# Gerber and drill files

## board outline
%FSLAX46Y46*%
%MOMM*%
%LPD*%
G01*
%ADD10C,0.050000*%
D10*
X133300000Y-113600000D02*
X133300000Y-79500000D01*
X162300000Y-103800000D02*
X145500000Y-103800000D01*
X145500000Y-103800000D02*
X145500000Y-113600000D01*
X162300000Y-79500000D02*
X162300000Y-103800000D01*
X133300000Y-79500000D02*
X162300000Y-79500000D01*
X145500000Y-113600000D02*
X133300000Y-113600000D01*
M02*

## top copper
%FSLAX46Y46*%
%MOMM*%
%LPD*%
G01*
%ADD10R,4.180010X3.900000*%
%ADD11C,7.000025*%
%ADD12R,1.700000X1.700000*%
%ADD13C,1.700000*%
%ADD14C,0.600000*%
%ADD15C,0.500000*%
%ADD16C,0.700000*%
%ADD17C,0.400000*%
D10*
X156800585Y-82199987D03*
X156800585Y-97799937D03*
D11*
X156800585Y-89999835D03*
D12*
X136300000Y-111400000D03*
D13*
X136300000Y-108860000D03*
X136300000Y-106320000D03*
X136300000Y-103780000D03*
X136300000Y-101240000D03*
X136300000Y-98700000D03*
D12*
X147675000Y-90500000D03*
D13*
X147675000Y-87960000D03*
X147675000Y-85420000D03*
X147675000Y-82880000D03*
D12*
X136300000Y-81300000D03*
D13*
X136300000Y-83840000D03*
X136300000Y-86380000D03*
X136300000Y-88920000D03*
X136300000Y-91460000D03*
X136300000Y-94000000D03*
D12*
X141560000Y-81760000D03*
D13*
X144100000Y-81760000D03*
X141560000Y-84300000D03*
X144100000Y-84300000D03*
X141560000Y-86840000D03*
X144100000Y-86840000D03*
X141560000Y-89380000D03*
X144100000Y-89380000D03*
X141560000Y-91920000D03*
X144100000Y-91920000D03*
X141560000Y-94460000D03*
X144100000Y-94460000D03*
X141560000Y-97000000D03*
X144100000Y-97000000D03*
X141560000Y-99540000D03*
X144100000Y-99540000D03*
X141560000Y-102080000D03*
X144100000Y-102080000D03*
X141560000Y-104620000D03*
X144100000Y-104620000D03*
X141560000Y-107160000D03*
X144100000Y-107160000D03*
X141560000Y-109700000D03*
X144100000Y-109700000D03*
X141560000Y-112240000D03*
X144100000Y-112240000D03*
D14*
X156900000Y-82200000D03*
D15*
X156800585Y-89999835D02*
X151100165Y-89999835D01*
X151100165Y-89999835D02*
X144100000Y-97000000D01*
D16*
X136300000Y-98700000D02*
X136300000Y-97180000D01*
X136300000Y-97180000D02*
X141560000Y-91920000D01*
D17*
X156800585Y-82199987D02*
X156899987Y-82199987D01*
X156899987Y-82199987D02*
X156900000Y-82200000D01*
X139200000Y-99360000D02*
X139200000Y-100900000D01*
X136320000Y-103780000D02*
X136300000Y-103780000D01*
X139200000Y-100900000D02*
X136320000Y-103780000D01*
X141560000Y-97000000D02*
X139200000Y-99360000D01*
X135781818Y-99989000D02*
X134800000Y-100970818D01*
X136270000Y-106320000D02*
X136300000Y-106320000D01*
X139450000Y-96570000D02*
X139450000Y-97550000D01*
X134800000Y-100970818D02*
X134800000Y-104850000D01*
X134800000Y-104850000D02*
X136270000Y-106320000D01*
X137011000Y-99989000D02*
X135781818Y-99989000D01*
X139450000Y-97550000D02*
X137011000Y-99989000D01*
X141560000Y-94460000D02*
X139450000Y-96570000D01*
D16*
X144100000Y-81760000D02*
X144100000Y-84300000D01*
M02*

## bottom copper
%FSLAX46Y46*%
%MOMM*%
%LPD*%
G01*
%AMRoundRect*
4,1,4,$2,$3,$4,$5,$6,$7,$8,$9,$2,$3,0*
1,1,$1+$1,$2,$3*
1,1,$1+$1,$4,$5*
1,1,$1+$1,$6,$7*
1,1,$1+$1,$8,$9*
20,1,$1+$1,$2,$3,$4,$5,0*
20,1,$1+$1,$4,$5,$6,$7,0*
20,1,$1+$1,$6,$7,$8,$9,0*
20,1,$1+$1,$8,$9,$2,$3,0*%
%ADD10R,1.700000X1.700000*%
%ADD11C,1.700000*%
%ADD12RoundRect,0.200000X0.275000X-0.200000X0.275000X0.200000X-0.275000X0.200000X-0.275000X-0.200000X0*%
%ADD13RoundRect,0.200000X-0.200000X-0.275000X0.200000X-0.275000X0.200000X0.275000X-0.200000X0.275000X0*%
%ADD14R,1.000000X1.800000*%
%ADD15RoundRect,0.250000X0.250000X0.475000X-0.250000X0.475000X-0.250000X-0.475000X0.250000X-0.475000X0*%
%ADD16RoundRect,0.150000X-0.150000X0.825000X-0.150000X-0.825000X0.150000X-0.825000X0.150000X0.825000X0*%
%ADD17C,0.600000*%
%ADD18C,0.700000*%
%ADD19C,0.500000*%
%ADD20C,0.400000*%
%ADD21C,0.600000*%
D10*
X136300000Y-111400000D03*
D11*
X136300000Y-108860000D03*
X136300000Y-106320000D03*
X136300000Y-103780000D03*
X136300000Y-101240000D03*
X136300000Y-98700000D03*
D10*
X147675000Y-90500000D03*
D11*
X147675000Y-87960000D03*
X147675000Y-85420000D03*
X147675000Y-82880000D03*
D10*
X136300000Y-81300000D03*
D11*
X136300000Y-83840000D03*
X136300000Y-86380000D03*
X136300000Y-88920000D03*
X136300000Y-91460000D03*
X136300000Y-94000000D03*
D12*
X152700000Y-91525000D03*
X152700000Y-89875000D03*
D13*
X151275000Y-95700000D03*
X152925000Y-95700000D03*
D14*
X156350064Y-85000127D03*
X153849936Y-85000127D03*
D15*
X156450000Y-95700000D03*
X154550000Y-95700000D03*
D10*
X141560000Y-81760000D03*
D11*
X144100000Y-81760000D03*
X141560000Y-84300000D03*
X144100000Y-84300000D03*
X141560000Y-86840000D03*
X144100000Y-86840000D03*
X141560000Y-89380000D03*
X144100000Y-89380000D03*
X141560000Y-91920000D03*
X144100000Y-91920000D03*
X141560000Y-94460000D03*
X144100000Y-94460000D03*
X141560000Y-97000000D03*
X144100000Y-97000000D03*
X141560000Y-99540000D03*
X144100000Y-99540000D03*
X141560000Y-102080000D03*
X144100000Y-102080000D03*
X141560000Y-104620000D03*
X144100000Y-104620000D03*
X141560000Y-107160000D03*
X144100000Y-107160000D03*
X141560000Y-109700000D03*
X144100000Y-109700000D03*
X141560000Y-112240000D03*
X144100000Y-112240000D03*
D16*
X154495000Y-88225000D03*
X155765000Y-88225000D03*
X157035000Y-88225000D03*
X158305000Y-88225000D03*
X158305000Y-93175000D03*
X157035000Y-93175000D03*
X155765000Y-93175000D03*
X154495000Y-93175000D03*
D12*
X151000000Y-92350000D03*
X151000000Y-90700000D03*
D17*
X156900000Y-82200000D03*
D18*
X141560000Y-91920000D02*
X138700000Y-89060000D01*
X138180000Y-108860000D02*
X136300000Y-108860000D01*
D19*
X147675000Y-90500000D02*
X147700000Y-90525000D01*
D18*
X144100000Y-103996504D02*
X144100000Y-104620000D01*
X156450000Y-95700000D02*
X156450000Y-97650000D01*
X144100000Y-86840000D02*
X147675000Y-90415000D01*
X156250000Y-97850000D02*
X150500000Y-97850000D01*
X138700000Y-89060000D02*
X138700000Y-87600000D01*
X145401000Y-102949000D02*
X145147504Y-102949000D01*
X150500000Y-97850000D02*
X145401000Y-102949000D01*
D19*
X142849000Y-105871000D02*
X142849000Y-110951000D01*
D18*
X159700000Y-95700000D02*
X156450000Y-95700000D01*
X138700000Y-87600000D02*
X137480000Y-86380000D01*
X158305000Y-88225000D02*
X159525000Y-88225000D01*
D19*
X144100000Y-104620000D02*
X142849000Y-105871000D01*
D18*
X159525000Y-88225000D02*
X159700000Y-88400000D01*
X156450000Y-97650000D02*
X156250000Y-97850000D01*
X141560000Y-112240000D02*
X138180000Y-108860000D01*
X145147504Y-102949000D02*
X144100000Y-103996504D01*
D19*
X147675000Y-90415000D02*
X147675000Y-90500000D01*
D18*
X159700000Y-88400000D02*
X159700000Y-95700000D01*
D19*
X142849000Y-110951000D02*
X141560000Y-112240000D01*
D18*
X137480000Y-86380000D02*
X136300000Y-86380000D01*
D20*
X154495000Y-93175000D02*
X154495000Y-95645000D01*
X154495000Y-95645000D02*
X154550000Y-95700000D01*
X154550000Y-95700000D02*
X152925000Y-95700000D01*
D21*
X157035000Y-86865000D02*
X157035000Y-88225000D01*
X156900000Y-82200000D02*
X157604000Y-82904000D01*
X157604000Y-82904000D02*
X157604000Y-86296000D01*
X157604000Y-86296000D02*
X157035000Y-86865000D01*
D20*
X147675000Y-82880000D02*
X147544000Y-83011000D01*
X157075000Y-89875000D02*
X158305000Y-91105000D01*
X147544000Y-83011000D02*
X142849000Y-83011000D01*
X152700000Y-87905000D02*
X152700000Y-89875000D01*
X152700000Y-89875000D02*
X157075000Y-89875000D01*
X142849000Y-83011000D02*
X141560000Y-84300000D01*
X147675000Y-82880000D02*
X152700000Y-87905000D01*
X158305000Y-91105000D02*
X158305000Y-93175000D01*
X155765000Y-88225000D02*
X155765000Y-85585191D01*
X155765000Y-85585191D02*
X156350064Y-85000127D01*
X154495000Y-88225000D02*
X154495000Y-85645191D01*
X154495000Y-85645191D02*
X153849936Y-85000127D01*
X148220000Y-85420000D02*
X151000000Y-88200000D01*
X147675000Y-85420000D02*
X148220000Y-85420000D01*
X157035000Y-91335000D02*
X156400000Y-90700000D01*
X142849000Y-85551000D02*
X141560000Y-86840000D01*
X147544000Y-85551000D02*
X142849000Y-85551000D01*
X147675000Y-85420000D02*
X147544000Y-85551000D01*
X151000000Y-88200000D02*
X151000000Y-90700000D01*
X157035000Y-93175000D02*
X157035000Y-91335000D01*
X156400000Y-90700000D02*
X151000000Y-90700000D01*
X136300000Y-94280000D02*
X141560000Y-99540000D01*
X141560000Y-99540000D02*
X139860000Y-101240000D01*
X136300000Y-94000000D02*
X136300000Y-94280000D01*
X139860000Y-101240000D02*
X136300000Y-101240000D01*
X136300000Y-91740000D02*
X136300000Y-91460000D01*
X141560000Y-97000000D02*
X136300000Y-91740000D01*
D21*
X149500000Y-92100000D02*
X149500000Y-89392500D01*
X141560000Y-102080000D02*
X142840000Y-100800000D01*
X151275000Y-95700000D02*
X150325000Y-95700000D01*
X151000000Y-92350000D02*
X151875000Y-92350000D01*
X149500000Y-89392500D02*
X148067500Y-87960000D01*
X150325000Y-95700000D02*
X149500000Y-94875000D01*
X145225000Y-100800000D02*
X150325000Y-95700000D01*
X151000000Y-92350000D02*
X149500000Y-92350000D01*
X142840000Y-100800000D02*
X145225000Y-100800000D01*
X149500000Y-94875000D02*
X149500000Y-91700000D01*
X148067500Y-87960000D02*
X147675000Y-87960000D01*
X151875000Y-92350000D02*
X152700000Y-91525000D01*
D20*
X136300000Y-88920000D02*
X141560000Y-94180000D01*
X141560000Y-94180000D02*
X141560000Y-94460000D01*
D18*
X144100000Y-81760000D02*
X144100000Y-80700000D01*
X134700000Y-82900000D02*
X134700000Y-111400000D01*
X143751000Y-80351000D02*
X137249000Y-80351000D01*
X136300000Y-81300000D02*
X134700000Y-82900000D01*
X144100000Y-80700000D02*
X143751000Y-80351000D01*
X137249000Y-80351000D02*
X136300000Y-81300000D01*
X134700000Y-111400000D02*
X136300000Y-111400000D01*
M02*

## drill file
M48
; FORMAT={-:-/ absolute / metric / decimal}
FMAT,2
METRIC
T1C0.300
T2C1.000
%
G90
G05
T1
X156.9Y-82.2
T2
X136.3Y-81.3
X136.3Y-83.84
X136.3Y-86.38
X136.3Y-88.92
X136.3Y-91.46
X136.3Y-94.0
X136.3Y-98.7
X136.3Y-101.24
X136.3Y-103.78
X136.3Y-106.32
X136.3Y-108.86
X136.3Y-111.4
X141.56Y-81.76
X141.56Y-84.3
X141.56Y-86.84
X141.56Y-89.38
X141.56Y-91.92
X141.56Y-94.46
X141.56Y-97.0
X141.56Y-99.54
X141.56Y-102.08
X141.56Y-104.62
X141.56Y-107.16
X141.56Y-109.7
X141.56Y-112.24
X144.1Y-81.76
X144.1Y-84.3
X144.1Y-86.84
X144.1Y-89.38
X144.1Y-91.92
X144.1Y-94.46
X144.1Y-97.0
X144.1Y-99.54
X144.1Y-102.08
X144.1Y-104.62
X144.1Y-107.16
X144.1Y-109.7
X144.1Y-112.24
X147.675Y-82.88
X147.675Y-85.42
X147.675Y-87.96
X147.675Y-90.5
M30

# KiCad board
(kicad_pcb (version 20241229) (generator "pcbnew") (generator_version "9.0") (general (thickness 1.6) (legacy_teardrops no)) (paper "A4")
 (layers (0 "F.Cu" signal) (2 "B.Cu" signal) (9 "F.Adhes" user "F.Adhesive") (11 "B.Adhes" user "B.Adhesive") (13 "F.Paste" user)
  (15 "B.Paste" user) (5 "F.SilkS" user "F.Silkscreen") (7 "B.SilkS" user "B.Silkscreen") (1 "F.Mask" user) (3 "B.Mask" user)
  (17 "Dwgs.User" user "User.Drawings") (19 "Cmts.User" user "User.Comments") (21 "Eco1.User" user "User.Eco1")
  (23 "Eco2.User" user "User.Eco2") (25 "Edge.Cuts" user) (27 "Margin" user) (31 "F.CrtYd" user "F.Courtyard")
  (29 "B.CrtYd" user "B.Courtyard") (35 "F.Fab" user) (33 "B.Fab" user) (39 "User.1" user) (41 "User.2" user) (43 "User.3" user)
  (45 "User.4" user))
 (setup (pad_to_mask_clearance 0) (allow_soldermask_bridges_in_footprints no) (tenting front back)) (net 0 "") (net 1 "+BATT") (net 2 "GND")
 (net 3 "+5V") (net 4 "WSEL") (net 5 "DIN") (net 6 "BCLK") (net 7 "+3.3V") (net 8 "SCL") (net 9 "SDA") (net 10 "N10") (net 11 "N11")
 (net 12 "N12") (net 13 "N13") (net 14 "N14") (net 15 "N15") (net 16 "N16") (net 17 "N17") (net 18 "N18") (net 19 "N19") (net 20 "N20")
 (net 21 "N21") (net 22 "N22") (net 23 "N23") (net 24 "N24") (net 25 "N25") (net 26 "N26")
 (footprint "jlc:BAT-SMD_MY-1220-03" (layer "F.Cu") (at 156.800585 89.999962 -90)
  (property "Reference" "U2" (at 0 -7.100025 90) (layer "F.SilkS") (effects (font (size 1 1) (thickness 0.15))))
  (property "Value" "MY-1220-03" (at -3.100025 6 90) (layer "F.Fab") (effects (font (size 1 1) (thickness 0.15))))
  (pad "1" smd rect (at -7.799975 0 270) (size 3.9 4.18001) (layers "F.Cu" "F.Mask" "F.Paste") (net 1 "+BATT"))
  (pad "2" smd rect (at 7.799975 0 270) (size 3.9 4.18001) (layers "F.Cu" "F.Mask" "F.Paste") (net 1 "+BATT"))
  (pad "3" smd circle (at -0.000127 0 270) (size 7.000025 7.000025) (layers "F.Cu" "F.Mask" "F.Paste") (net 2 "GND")))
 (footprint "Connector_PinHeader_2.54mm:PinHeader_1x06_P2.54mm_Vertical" (layer "F.Cu") (at 136.3 111.4 180)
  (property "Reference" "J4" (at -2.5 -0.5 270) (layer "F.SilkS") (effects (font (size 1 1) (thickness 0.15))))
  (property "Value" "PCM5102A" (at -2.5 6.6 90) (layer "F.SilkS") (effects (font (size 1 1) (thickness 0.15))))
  (pad "1" thru_hole rect (at 0 0 180) (size 1.7 1.7) (drill 1) (layers "*.Cu" "*.Mask") (remove_unused_layers no) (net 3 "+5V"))
  (pad "2" thru_hole circle (at 0 2.54 180) (size 1.7 1.7) (drill 1) (layers "*.Cu" "*.Mask") (remove_unused_layers no) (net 2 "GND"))
  (pad "3" thru_hole circle (at 0 5.08 180) (size 1.7 1.7) (drill 1) (layers "*.Cu" "*.Mask") (remove_unused_layers no) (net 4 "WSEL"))
  (pad "4" thru_hole circle (at 0 7.62 180) (size 1.7 1.7) (drill 1) (layers "*.Cu" "*.Mask") (remove_unused_layers no) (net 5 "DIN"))
  (pad "5" thru_hole circle (at 0 10.16 180) (size 1.7 1.7) (drill 1) (layers "*.Cu" "*.Mask") (remove_unused_layers no) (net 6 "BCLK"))
  (pad "6" thru_hole circle (at 0 12.7 180) (size 1.7 1.7) (drill 1) (layers "*.Cu" "*.Mask") (remove_unused_layers no) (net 2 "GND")))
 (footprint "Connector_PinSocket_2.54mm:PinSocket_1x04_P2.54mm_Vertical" (layer "F.Cu") (at 147.675 90.5 180)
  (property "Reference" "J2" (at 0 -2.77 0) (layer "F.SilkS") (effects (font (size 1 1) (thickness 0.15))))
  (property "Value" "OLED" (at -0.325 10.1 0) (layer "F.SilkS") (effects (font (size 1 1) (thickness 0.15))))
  (pad "1" thru_hole rect (at 0 0 180) (size 1.7 1.7) (drill 1) (layers "*.Cu" "*.Mask") (remove_unused_layers no) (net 2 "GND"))
  (pad "2" thru_hole circle (at 0 2.54 180) (size 1.7 1.7) (drill 1) (layers "*.Cu" "*.Mask") (remove_unused_layers no) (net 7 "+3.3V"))
  (pad "3" thru_hole circle (at 0 5.08 180) (size 1.7 1.7) (drill 1) (layers "*.Cu" "*.Mask") (remove_unused_layers no) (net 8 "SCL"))
  (pad "4" thru_hole circle (at 0 7.62 180) (size 1.7 1.7) (drill 1) (layers "*.Cu" "*.Mask") (remove_unused_layers no) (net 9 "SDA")))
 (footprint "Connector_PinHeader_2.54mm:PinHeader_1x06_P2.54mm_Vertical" (layer "F.Cu") (at 136.3 81.3)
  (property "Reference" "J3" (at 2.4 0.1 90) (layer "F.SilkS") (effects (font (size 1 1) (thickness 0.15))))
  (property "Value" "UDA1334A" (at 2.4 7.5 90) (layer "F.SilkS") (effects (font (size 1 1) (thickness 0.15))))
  (pad "1" thru_hole rect (at 0 0) (size 1.7 1.7) (drill 1) (layers "*.Cu" "*.Mask") (remove_unused_layers no) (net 3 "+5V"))
  (pad "2" thru_hole circle (at 0 2.54) (size 1.7 1.7) (drill 1) (layers "*.Cu" "*.Mask") (remove_unused_layers no) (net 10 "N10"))
  (pad "3" thru_hole circle (at 0 5.08) (size 1.7 1.7) (drill 1) (layers "*.Cu" "*.Mask") (remove_unused_layers no) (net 2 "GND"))
  (pad "4" thru_hole circle (at 0 7.62) (size 1.7 1.7) (drill 1) (layers "*.Cu" "*.Mask") (remove_unused_layers no) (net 4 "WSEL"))
  (pad "5" thru_hole circle (at 0 10.16) (size 1.7 1.7) (drill 1) (layers "*.Cu" "*.Mask") (remove_unused_layers no) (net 5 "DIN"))
  (pad "6" thru_hole circle (at 0 12.7) (size 1.7 1.7) (drill 1) (layers "*.Cu" "*.Mask") (remove_unused_layers no) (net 6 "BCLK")))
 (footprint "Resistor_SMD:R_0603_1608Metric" (layer "B.Cu") (at 152.7 90.7 90)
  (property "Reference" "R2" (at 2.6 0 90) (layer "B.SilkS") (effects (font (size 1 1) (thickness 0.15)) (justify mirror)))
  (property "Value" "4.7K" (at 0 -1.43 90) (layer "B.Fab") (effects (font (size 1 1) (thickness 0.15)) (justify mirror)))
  (pad "1" smd roundrect (at -0.825 0 90) (size 0.8 0.95) (layers "B.Cu" "B.Mask" "B.Paste") (roundrect_rratio 0.25) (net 7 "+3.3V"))
  (pad "2" smd roundrect (at 0.825 0 90) (size 0.8 0.95) (layers "B.Cu" "B.Mask" "B.Paste") (roundrect_rratio 0.25) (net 9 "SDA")))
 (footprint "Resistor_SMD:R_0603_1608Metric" (layer "B.Cu") (at 152.1 95.7)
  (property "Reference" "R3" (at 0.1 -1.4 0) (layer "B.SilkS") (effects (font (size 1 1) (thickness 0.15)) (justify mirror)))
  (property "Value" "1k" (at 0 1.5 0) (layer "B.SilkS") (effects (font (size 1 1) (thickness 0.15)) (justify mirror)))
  (pad "1" smd roundrect (at -0.825 0) (size 0.8 0.95) (layers "B.Cu" "B.Mask" "B.Paste") (roundrect_rratio 0.25) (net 7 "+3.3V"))
  (pad "2" smd roundrect (at 0.825 0) (size 0.8 0.95) (layers "B.Cu" "B.Mask" "B.Paste") (roundrect_rratio 0.25) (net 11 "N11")))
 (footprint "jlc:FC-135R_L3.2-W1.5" (layer "B.Cu") (at 155.1 85 180)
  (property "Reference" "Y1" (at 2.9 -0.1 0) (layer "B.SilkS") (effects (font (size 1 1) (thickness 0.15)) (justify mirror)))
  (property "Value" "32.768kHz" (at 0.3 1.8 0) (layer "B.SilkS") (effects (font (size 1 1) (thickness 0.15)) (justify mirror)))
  (pad "1" smd rect (at -1.250064 -0.000127 90) (size 1.8 1) (layers "B.Cu" "B.Mask" "B.Paste") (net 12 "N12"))
  (pad "2" smd rect (at 1.250064 -0.000127 90) (size 1.8 1) (layers "B.Cu" "B.Mask" "B.Paste") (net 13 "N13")))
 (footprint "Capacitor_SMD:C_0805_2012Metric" (layer "B.Cu") (at 155.5 95.7 180)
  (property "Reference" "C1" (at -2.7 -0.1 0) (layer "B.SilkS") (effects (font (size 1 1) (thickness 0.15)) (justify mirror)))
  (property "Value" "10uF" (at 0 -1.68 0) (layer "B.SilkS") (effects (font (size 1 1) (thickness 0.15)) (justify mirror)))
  (pad "1" smd roundrect (at -0.95 0 180) (size 1 1.45) (layers "B.Cu" "B.Mask" "B.Paste") (roundrect_rratio 0.25) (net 2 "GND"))
  (pad "2" smd roundrect (at 0.95 0 180) (size 1 1.45) (layers "B.Cu" "B.Mask" "B.Paste") (roundrect_rratio 0.25) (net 11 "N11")))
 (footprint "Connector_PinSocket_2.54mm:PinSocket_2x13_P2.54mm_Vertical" (layer "B.Cu") (at 141.56 81.76 180)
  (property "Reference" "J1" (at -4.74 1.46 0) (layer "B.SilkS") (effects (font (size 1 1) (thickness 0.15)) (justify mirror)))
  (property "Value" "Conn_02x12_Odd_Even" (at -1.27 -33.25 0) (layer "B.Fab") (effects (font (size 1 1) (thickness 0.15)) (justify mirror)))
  (pad "1" thru_hole rect (at 0 0 180) (size 1.7 1.7) (drill 1) (layers "*.Cu" "*.Mask") (remove_unused_layers no) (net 7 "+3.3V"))
  (pad "2" thru_hole circle (at -2.54 0 180) (size 1.7 1.7) (drill 1) (layers "*.Cu" "*.Mask") (remove_unused_layers no) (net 3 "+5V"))
  (pad "3" thru_hole circle (at 0 -2.54 180) (size 1.7 1.7) (drill 1) (layers "*.Cu" "*.Mask") (remove_unused_layers no) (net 9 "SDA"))
  (pad "4" thru_hole circle (at -2.54 -2.54 180) (size 1.7 1.7) (drill 1) (layers "*.Cu" "*.Mask") (remove_unused_layers no) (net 3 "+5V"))
  (pad "5" thru_hole circle (at 0 -5.08 180) (size 1.7 1.7) (drill 1) (layers "*.Cu" "*.Mask") (remove_unused_layers no) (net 8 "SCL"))
  (pad "6" thru_hole circle (at -2.54 -5.08 180) (size 1.7 1.7) (drill 1) (layers "*.Cu" "*.Mask") (remove_unused_layers no) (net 2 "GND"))
  (pad "7" thru_hole circle (at 0 -7.62 180) (size 1.7 1.7) (drill 1) (layers "*.Cu" "*.Mask") (remove_unused_layers no) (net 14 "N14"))
  (pad "8" thru_hole circle (at -2.54 -7.62 180) (size 1.7 1.7) (drill 1) (layers "*.Cu" "*.Mask") (remove_unused_layers no) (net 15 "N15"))
  (pad "9" thru_hole circle (at 0 -10.16 180) (size 1.7 1.7) (drill 1) (layers "*.Cu" "*.Mask") (remove_unused_layers no) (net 2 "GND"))
  (pad "10" thru_hole circle (at -2.54 -10.16 180) (size 1.7 1.7) (drill 1) (layers "*.Cu" "*.Mask") (remove_unused_layers no)
   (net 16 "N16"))
  (pad "11" thru_hole circle (at 0 -12.7 180) (size 1.7 1.7) (drill 1) (layers "*.Cu" "*.Mask") (remove_unused_layers no) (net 4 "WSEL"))
  (pad "12" thru_hole circle (at -2.54 -12.7 180) (size 1.7 1.7) (drill 1) (layers "*.Cu" "*.Mask") (remove_unused_layers no) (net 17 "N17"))
  (pad "13" thru_hole circle (at 0 -15.24 180) (size 1.7 1.7) (drill 1) (layers "*.Cu" "*.Mask") (remove_unused_layers no) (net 5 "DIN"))
  (pad "14" thru_hole circle (at -2.54 -15.24 180) (size 1.7 1.7) (drill 1) (layers "*.Cu" "*.Mask") (remove_unused_layers no) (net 2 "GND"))
  (pad "15" thru_hole circle (at 0 -17.78 180) (size 1.7 1.7) (drill 1) (layers "*.Cu" "*.Mask") (remove_unused_layers no) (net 6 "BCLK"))
  (pad "16" thru_hole circle (at -2.54 -17.78 180) (size 1.7 1.7) (drill 1) (layers "*.Cu" "*.Mask") (remove_unused_layers no)
   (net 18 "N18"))
  (pad "17" thru_hole circle (at 0 -20.32 180) (size 1.7 1.7) (drill 1) (layers "*.Cu" "*.Mask") (remove_unused_layers no) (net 7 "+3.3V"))
  (pad "18" thru_hole circle (at -2.54 -20.32 180) (size 1.7 1.7) (drill 1) (layers "*.Cu" "*.Mask") (remove_unused_layers no)
   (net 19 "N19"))
  (pad "19" thru_hole circle (at 0 -22.86 180) (size 1.7 1.7) (drill 1) (layers "*.Cu" "*.Mask") (remove_unused_layers no) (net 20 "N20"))
  (pad "20" thru_hole circle (at -2.54 -22.86 180) (size 1.7 1.7) (drill 1) (layers "*.Cu" "*.Mask") (remove_unused_layers no) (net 2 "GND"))
  (pad "21" thru_hole circle (at 0 -25.4 180) (size 1.7 1.7) (drill 1) (layers "*.Cu" "*.Mask") (remove_unused_layers no) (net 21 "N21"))
  (pad "22" thru_hole circle (at -2.54 -25.4 180) (size 1.7 1.7) (drill 1) (layers "*.Cu" "*.Mask") (remove_unused_layers no) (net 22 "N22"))
  (pad "23" thru_hole circle (at 0 -27.94 180) (size 1.7 1.7) (drill 1) (layers "*.Cu" "*.Mask") (remove_unused_layers no) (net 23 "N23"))
  (pad "24" thru_hole circle (at -2.54 -27.94 180) (size 1.7 1.7) (drill 1) (layers "*.Cu" "*.Mask") (remove_unused_layers no)
   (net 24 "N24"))
  (pad "25" thru_hole circle (at 0 -30.48 180) (size 1.7 1.7) (drill 1) (layers "*.Cu" "*.Mask") (remove_unused_layers no) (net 2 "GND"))
  (pad "26" thru_hole circle (at -2.54 -30.48 180) (size 1.7 1.7) (drill 1) (layers "*.Cu" "*.Mask") (remove_unused_layers no)
   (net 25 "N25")))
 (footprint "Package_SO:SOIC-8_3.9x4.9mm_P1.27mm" (layer "B.Cu") (at 156.4 90.7 -90)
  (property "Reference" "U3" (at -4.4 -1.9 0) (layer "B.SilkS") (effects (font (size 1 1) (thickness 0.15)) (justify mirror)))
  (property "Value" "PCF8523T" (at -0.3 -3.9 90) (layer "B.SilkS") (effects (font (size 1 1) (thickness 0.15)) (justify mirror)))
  (pad "1" smd roundrect (at -2.475 1.905 270) (size 1.95 0.6) (layers "B.Cu" "B.Mask" "B.Paste") (roundrect_rratio 0.25) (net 13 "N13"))
  (pad "2" smd roundrect (at -2.475 0.635 270) (size 1.95 0.6) (layers "B.Cu" "B.Mask" "B.Paste") (roundrect_rratio 0.25) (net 12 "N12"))
  (pad "3" smd roundrect (at -2.475 -0.635 270) (size 1.95 0.6) (layers "B.Cu" "B.Mask" "B.Paste") (roundrect_rratio 0.25) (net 1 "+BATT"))
  (pad "4" smd roundrect (at -2.475 -1.905 270) (size 1.95 0.6) (layers "B.Cu" "B.Mask" "B.Paste") (roundrect_rratio 0.25) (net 2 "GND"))
  (pad "5" smd roundrect (at 2.475 -1.905 270) (size 1.95 0.6) (layers "B.Cu" "B.Mask" "B.Paste") (roundrect_rratio 0.25) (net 9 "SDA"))
  (pad "6" smd roundrect (at 2.475 -0.635 270) (size 1.95 0.6) (layers "B.Cu" "B.Mask" "B.Paste") (roundrect_rratio 0.25) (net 8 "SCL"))
  (pad "7" smd roundrect (at 2.475 0.635 270) (size 1.95 0.6) (layers "B.Cu" "B.Mask" "B.Paste") (roundrect_rratio 0.25) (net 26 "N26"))
  (pad "8" smd roundrect (at 2.475 1.905 270) (size 1.95 0.6) (layers "B.Cu" "B.Mask" "B.Paste") (roundrect_rratio 0.25) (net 11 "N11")))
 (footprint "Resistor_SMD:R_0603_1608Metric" (layer "B.Cu") (at 151 91.525 90)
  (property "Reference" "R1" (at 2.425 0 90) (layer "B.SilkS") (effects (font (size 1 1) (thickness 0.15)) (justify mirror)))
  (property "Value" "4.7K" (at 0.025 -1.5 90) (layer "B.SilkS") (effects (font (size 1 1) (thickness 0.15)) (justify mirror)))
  (pad "1" smd roundrect (at -0.825 0 90) (size 0.8 0.95) (layers "B.Cu" "B.Mask" "B.Paste") (roundrect_rratio 0.25) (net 7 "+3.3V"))
  (pad "2" smd roundrect (at 0.825 0 90) (size 0.8 0.95) (layers "B.Cu" "B.Mask" "B.Paste") (roundrect_rratio 0.25) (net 8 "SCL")))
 (gr_line (start 133.3 113.6) (end 133.3 79.5) (stroke (width 0.05) (type default)) (layer "Edge.Cuts"))
 (gr_line (start 162.3 103.8) (end 145.5 103.8) (stroke (width 0.05) (type default)) (layer "Edge.Cuts"))
 (gr_line (start 145.5 103.8) (end 145.5 113.6) (stroke (width 0.05) (type default)) (layer "Edge.Cuts"))
 (gr_line (start 162.3 79.5) (end 162.3 103.8) (stroke (width 0.05) (type default)) (layer "Edge.Cuts"))
 (gr_line (start 133.3 79.5) (end 162.3 79.5) (stroke (width 0.05) (type default)) (layer "Edge.Cuts"))
 (gr_line (start 145.5 113.6) (end 133.3 113.6) (stroke (width 0.05) (type default)) (layer "Edge.Cuts"))
 (segment (start 156.800585 89.999835) (end 151.100165 89.999835) (width 0.5) (layer "F.Cu") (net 2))
 (segment (start 151.100165 89.999835) (end 144.1 97) (width 0.5) (layer "F.Cu") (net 2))
 (segment (start 136.3 98.7) (end 136.3 97.18) (width 0.7) (layer "F.Cu") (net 2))
 (segment (start 136.3 97.18) (end 141.56 91.92) (width 0.7) (layer "F.Cu") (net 2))
 (segment (start 141.56 91.92) (end 138.7 89.06) (width 0.7) (layer "B.Cu") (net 2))
 (segment (start 138.18 108.86) (end 136.3 108.86) (width 0.7) (layer "B.Cu") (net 2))
 (segment (start 147.675 90.5) (end 147.7 90.525) (width 0.5) (layer "B.Cu") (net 2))
 (segment (start 144.1 103.996504) (end 144.1 104.62) (width 0.7) (layer "B.Cu") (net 2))
 (segment (start 156.45 95.7) (end 156.45 97.65) (width 0.7) (layer "B.Cu") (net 2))
 (segment (start 144.1 86.84) (end 147.675 90.415) (width 0.7) (layer "B.Cu") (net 2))
 (segment (start 156.25 97.85) (end 150.5 97.85) (width 0.7) (layer "B.Cu") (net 2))
 (segment (start 138.7 89.06) (end 138.7 87.6) (width 0.7) (layer "B.Cu") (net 2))
 (segment (start 145.401 102.949) (end 145.147504 102.949) (width 0.7) (layer "B.Cu") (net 2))
 (segment (start 150.5 97.85) (end 145.401 102.949) (width 0.7) (layer "B.Cu") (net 2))
 (segment (start 142.849 105.871) (end 142.849 110.951) (width 0.5) (layer "B.Cu") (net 2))
 (segment (start 159.7 95.7) (end 156.45 95.7) (width 0.7) (layer "B.Cu") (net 2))
 (segment (start 138.7 87.6) (end 137.48 86.38) (width 0.7) (layer "B.Cu") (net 2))
 (segment (start 158.305 88.225) (end 159.525 88.225) (width 0.7) (layer "B.Cu") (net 2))
 (segment (start 144.1 104.62) (end 142.849 105.871) (width 0.5) (layer "B.Cu") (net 2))
 (segment (start 159.525 88.225) (end 159.7 88.4) (width 0.7) (layer "B.Cu") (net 2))
 (segment (start 156.45 97.65) (end 156.25 97.85) (width 0.7) (layer "B.Cu") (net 2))
 (segment (start 141.56 112.24) (end 138.18 108.86) (width 0.7) (layer "B.Cu") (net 2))
 (segment (start 145.147504 102.949) (end 144.1 103.996504) (width 0.7) (layer "B.Cu") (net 2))
 (segment (start 147.675 90.415) (end 147.675 90.5) (width 0.5) (layer "B.Cu") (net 2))
 (segment (start 159.7 88.4) (end 159.7 95.7) (width 0.7) (layer "B.Cu") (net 2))
 (segment (start 142.849 110.951) (end 141.56 112.24) (width 0.5) (layer "B.Cu") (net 2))
 (segment (start 137.48 86.38) (end 136.3 86.38) (width 0.7) (layer "B.Cu") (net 2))
 (segment (start 154.495 93.175) (end 154.495 95.645) (width 0.4) (layer "B.Cu") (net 11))
 (segment (start 154.495 95.645) (end 154.55 95.7) (width 0.4) (layer "B.Cu") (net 11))
 (segment (start 154.55 95.7) (end 152.925 95.7) (width 0.4) (layer "B.Cu") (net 11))
 (segment (start 156.800585 82.199987) (end 156.899987 82.199987) (width 0.4) (layer "F.Cu") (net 1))
 (segment (start 156.899987 82.199987) (end 156.9 82.2) (width 0.4) (layer "F.Cu") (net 1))
 (via (at 156.9 82.2) (size 0.6) (drill 0.3) (layers "F.Cu" "B.Cu") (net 1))
 (segment (start 157.035 86.865) (end 157.035 88.225) (width 0.6) (layer "B.Cu") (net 1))
 (segment (start 156.9 82.2) (end 157.604 82.904) (width 0.6) (layer "B.Cu") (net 1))
 (segment (start 157.604 82.904) (end 157.604 86.296) (width 0.6) (layer "B.Cu") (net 1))
 (segment (start 157.604 86.296) (end 157.035 86.865) (width 0.6) (layer "B.Cu") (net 1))
 (segment (start 147.675 82.88) (end 147.544 83.011) (width 0.4) (layer "B.Cu") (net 9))
 (segment (start 157.075 89.875) (end 158.305 91.105) (width 0.4) (layer "B.Cu") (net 9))
 (segment (start 147.544 83.011) (end 142.849 83.011) (width 0.4) (layer "B.Cu") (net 9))
 (segment (start 152.7 87.905) (end 152.7 89.875) (width 0.4) (layer "B.Cu") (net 9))
 (segment (start 152.7 89.875) (end 157.075 89.875) (width 0.4) (layer "B.Cu") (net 9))
 (segment (start 142.849 83.011) (end 141.56 84.3) (width 0.4) (layer "B.Cu") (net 9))
 (segment (start 147.675 82.88) (end 152.7 87.905) (width 0.4) (layer "B.Cu") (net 9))
 (segment (start 158.305 91.105) (end 158.305 93.175) (width 0.4) (layer "B.Cu") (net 9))
 (segment (start 155.765 88.225) (end 155.765 85.585191) (width 0.4) (layer "B.Cu") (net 12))
 (segment (start 155.765 85.585191) (end 156.350064 85.000127) (width 0.4) (layer "B.Cu") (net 12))
 (segment (start 154.495 88.225) (end 154.495 85.645191) (width 0.4) (layer "B.Cu") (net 13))
 (segment (start 154.495 85.645191) (end 153.849936 85.000127) (width 0.4) (layer "B.Cu") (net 13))
 (segment (start 148.22 85.42) (end 151 88.2) (width 0.4) (layer "B.Cu") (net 8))
 (segment (start 147.675 85.42) (end 148.22 85.42) (width 0.4) (layer "B.Cu") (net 8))
 (segment (start 157.035 91.335) (end 156.4 90.7) (width 0.4) (layer "B.Cu") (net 8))
 (segment (start 142.849 85.551) (end 141.56 86.84) (width 0.4) (layer "B.Cu") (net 8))
 (segment (start 147.544 85.551) (end 142.849 85.551) (width 0.4) (layer "B.Cu") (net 8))
 (segment (start 147.675 85.42) (end 147.544 85.551) (width 0.4) (layer "B.Cu") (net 8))
 (segment (start 151 88.2) (end 151 90.7) (width 0.4) (layer "B.Cu") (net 8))
 (segment (start 157.035 93.175) (end 157.035 91.335) (width 0.4) (layer "B.Cu") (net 8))
 (segment (start 156.4 90.7) (end 151 90.7) (width 0.4) (layer "B.Cu") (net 8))
 (segment (start 136.3 94.28) (end 141.56 99.54) (width 0.4) (layer "B.Cu") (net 6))
 (segment (start 141.56 99.54) (end 139.86 101.24) (width 0.4) (layer "B.Cu") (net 6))
 (segment (start 136.3 94) (end 136.3 94.28) (width 0.4) (layer "B.Cu") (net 6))
 (segment (start 139.86 101.24) (end 136.3 101.24) (width 0.4) (layer "B.Cu") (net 6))
 (segment (start 139.2 99.36) (end 139.2 100.9) (width 0.4) (layer "F.Cu") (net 5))
 (segment (start 136.32 103.78) (end 136.3 103.78) (width 0.4) (layer "F.Cu") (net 5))
 (segment (start 139.2 100.9) (end 136.32 103.78) (width 0.4) (layer "F.Cu") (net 5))
 (segment (start 141.56 97) (end 139.2 99.36) (width 0.4) (layer "F.Cu") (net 5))
 (segment (start 136.3 91.74) (end 136.3 91.46) (width 0.4) (layer "B.Cu") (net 5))
 (segment (start 141.56 97) (end 136.3 91.74) (width 0.4) (layer "B.Cu") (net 5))
 (segment (start 149.5 92.1) (end 149.5 89.3925) (width 0.6) (layer "B.Cu") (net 7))
 (segment (start 141.56 102.08) (end 142.84 100.8) (width 0.6) (layer "B.Cu") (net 7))
 (segment (start 151.275 95.7) (end 150.325 95.7) (width 0.6) (layer "B.Cu") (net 7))
 (segment (start 151 92.35) (end 151.875 92.35) (width 0.6) (layer "B.Cu") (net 7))
 (segment (start 149.5 89.3925) (end 148.0675 87.96) (width 0.6) (layer "B.Cu") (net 7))
 (segment (start 150.325 95.7) (end 149.5 94.875) (width 0.6) (layer "B.Cu") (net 7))
 (segment (start 145.225 100.8) (end 150.325 95.7) (width 0.6) (layer "B.Cu") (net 7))
 (segment (start 151 92.35) (end 149.5 92.35) (width 0.6) (layer "B.Cu") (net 7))
 (segment (start 142.84 100.8) (end 145.225 100.8) (width 0.6) (layer "B.Cu") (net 7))
 (segment (start 149.5 94.875) (end 149.5 91.7) (width 0.6) (layer "B.Cu") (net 7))
 (segment (start 148.0675 87.96) (end 147.675 87.96) (width 0.6) (layer "B.Cu") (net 7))
 (segment (start 151.875 92.35) (end 152.7 91.525) (width 0.6) (layer "B.Cu") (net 7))
 (segment (start 135.781818 99.989) (end 134.8 100.970818) (width 0.4) (layer "F.Cu") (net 4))
 (segment (start 136.27 106.32) (end 136.3 106.32) (width 0.4) (layer "F.Cu") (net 4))
 (segment (start 139.45 96.57) (end 139.45 97.55) (width 0.4) (layer "F.Cu") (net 4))
 (segment (start 134.8 100.970818) (end 134.8 104.85) (width 0.4) (layer "F.Cu") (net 4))
 (segment (start 134.8 104.85) (end 136.27 106.32) (width 0.4) (layer "F.Cu") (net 4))
 (segment (start 137.011 99.989) (end 135.781818 99.989) (width 0.4) (layer "F.Cu") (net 4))
 (segment (start 139.45 97.55) (end 137.011 99.989) (width 0.4) (layer "F.Cu") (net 4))
 (segment (start 141.56 94.46) (end 139.45 96.57) (width 0.4) (layer "F.Cu") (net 4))
 (segment (start 136.3 88.92) (end 141.56 94.18) (width 0.4) (layer "B.Cu") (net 4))
 (segment (start 141.56 94.18) (end 141.56 94.46) (width 0.4) (layer "B.Cu") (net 4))
 (segment (start 144.1 81.76) (end 144.1 84.3) (width 0.7) (layer "F.Cu") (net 3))
 (segment (start 144.1 81.76) (end 144.1 80.7) (width 0.7) (layer "B.Cu") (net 3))
 (segment (start 134.7 82.9) (end 134.7 111.4) (width 0.7) (layer "B.Cu") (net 3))
 (segment (start 143.751 80.351) (end 137.249 80.351) (width 0.7) (layer "B.Cu") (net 3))
 (segment (start 136.3 81.3) (end 134.7 82.9) (width 0.7) (layer "B.Cu") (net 3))
 (segment (start 144.1 80.7) (end 143.751 80.351) (width 0.7) (layer "B.Cu") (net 3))
 (segment (start 137.249 80.351) (end 136.3 81.3) (width 0.7) (layer "B.Cu") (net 3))
 (segment (start 134.7 111.4) (end 136.3 111.4) (width 0.7) (layer "B.Cu") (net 3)))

